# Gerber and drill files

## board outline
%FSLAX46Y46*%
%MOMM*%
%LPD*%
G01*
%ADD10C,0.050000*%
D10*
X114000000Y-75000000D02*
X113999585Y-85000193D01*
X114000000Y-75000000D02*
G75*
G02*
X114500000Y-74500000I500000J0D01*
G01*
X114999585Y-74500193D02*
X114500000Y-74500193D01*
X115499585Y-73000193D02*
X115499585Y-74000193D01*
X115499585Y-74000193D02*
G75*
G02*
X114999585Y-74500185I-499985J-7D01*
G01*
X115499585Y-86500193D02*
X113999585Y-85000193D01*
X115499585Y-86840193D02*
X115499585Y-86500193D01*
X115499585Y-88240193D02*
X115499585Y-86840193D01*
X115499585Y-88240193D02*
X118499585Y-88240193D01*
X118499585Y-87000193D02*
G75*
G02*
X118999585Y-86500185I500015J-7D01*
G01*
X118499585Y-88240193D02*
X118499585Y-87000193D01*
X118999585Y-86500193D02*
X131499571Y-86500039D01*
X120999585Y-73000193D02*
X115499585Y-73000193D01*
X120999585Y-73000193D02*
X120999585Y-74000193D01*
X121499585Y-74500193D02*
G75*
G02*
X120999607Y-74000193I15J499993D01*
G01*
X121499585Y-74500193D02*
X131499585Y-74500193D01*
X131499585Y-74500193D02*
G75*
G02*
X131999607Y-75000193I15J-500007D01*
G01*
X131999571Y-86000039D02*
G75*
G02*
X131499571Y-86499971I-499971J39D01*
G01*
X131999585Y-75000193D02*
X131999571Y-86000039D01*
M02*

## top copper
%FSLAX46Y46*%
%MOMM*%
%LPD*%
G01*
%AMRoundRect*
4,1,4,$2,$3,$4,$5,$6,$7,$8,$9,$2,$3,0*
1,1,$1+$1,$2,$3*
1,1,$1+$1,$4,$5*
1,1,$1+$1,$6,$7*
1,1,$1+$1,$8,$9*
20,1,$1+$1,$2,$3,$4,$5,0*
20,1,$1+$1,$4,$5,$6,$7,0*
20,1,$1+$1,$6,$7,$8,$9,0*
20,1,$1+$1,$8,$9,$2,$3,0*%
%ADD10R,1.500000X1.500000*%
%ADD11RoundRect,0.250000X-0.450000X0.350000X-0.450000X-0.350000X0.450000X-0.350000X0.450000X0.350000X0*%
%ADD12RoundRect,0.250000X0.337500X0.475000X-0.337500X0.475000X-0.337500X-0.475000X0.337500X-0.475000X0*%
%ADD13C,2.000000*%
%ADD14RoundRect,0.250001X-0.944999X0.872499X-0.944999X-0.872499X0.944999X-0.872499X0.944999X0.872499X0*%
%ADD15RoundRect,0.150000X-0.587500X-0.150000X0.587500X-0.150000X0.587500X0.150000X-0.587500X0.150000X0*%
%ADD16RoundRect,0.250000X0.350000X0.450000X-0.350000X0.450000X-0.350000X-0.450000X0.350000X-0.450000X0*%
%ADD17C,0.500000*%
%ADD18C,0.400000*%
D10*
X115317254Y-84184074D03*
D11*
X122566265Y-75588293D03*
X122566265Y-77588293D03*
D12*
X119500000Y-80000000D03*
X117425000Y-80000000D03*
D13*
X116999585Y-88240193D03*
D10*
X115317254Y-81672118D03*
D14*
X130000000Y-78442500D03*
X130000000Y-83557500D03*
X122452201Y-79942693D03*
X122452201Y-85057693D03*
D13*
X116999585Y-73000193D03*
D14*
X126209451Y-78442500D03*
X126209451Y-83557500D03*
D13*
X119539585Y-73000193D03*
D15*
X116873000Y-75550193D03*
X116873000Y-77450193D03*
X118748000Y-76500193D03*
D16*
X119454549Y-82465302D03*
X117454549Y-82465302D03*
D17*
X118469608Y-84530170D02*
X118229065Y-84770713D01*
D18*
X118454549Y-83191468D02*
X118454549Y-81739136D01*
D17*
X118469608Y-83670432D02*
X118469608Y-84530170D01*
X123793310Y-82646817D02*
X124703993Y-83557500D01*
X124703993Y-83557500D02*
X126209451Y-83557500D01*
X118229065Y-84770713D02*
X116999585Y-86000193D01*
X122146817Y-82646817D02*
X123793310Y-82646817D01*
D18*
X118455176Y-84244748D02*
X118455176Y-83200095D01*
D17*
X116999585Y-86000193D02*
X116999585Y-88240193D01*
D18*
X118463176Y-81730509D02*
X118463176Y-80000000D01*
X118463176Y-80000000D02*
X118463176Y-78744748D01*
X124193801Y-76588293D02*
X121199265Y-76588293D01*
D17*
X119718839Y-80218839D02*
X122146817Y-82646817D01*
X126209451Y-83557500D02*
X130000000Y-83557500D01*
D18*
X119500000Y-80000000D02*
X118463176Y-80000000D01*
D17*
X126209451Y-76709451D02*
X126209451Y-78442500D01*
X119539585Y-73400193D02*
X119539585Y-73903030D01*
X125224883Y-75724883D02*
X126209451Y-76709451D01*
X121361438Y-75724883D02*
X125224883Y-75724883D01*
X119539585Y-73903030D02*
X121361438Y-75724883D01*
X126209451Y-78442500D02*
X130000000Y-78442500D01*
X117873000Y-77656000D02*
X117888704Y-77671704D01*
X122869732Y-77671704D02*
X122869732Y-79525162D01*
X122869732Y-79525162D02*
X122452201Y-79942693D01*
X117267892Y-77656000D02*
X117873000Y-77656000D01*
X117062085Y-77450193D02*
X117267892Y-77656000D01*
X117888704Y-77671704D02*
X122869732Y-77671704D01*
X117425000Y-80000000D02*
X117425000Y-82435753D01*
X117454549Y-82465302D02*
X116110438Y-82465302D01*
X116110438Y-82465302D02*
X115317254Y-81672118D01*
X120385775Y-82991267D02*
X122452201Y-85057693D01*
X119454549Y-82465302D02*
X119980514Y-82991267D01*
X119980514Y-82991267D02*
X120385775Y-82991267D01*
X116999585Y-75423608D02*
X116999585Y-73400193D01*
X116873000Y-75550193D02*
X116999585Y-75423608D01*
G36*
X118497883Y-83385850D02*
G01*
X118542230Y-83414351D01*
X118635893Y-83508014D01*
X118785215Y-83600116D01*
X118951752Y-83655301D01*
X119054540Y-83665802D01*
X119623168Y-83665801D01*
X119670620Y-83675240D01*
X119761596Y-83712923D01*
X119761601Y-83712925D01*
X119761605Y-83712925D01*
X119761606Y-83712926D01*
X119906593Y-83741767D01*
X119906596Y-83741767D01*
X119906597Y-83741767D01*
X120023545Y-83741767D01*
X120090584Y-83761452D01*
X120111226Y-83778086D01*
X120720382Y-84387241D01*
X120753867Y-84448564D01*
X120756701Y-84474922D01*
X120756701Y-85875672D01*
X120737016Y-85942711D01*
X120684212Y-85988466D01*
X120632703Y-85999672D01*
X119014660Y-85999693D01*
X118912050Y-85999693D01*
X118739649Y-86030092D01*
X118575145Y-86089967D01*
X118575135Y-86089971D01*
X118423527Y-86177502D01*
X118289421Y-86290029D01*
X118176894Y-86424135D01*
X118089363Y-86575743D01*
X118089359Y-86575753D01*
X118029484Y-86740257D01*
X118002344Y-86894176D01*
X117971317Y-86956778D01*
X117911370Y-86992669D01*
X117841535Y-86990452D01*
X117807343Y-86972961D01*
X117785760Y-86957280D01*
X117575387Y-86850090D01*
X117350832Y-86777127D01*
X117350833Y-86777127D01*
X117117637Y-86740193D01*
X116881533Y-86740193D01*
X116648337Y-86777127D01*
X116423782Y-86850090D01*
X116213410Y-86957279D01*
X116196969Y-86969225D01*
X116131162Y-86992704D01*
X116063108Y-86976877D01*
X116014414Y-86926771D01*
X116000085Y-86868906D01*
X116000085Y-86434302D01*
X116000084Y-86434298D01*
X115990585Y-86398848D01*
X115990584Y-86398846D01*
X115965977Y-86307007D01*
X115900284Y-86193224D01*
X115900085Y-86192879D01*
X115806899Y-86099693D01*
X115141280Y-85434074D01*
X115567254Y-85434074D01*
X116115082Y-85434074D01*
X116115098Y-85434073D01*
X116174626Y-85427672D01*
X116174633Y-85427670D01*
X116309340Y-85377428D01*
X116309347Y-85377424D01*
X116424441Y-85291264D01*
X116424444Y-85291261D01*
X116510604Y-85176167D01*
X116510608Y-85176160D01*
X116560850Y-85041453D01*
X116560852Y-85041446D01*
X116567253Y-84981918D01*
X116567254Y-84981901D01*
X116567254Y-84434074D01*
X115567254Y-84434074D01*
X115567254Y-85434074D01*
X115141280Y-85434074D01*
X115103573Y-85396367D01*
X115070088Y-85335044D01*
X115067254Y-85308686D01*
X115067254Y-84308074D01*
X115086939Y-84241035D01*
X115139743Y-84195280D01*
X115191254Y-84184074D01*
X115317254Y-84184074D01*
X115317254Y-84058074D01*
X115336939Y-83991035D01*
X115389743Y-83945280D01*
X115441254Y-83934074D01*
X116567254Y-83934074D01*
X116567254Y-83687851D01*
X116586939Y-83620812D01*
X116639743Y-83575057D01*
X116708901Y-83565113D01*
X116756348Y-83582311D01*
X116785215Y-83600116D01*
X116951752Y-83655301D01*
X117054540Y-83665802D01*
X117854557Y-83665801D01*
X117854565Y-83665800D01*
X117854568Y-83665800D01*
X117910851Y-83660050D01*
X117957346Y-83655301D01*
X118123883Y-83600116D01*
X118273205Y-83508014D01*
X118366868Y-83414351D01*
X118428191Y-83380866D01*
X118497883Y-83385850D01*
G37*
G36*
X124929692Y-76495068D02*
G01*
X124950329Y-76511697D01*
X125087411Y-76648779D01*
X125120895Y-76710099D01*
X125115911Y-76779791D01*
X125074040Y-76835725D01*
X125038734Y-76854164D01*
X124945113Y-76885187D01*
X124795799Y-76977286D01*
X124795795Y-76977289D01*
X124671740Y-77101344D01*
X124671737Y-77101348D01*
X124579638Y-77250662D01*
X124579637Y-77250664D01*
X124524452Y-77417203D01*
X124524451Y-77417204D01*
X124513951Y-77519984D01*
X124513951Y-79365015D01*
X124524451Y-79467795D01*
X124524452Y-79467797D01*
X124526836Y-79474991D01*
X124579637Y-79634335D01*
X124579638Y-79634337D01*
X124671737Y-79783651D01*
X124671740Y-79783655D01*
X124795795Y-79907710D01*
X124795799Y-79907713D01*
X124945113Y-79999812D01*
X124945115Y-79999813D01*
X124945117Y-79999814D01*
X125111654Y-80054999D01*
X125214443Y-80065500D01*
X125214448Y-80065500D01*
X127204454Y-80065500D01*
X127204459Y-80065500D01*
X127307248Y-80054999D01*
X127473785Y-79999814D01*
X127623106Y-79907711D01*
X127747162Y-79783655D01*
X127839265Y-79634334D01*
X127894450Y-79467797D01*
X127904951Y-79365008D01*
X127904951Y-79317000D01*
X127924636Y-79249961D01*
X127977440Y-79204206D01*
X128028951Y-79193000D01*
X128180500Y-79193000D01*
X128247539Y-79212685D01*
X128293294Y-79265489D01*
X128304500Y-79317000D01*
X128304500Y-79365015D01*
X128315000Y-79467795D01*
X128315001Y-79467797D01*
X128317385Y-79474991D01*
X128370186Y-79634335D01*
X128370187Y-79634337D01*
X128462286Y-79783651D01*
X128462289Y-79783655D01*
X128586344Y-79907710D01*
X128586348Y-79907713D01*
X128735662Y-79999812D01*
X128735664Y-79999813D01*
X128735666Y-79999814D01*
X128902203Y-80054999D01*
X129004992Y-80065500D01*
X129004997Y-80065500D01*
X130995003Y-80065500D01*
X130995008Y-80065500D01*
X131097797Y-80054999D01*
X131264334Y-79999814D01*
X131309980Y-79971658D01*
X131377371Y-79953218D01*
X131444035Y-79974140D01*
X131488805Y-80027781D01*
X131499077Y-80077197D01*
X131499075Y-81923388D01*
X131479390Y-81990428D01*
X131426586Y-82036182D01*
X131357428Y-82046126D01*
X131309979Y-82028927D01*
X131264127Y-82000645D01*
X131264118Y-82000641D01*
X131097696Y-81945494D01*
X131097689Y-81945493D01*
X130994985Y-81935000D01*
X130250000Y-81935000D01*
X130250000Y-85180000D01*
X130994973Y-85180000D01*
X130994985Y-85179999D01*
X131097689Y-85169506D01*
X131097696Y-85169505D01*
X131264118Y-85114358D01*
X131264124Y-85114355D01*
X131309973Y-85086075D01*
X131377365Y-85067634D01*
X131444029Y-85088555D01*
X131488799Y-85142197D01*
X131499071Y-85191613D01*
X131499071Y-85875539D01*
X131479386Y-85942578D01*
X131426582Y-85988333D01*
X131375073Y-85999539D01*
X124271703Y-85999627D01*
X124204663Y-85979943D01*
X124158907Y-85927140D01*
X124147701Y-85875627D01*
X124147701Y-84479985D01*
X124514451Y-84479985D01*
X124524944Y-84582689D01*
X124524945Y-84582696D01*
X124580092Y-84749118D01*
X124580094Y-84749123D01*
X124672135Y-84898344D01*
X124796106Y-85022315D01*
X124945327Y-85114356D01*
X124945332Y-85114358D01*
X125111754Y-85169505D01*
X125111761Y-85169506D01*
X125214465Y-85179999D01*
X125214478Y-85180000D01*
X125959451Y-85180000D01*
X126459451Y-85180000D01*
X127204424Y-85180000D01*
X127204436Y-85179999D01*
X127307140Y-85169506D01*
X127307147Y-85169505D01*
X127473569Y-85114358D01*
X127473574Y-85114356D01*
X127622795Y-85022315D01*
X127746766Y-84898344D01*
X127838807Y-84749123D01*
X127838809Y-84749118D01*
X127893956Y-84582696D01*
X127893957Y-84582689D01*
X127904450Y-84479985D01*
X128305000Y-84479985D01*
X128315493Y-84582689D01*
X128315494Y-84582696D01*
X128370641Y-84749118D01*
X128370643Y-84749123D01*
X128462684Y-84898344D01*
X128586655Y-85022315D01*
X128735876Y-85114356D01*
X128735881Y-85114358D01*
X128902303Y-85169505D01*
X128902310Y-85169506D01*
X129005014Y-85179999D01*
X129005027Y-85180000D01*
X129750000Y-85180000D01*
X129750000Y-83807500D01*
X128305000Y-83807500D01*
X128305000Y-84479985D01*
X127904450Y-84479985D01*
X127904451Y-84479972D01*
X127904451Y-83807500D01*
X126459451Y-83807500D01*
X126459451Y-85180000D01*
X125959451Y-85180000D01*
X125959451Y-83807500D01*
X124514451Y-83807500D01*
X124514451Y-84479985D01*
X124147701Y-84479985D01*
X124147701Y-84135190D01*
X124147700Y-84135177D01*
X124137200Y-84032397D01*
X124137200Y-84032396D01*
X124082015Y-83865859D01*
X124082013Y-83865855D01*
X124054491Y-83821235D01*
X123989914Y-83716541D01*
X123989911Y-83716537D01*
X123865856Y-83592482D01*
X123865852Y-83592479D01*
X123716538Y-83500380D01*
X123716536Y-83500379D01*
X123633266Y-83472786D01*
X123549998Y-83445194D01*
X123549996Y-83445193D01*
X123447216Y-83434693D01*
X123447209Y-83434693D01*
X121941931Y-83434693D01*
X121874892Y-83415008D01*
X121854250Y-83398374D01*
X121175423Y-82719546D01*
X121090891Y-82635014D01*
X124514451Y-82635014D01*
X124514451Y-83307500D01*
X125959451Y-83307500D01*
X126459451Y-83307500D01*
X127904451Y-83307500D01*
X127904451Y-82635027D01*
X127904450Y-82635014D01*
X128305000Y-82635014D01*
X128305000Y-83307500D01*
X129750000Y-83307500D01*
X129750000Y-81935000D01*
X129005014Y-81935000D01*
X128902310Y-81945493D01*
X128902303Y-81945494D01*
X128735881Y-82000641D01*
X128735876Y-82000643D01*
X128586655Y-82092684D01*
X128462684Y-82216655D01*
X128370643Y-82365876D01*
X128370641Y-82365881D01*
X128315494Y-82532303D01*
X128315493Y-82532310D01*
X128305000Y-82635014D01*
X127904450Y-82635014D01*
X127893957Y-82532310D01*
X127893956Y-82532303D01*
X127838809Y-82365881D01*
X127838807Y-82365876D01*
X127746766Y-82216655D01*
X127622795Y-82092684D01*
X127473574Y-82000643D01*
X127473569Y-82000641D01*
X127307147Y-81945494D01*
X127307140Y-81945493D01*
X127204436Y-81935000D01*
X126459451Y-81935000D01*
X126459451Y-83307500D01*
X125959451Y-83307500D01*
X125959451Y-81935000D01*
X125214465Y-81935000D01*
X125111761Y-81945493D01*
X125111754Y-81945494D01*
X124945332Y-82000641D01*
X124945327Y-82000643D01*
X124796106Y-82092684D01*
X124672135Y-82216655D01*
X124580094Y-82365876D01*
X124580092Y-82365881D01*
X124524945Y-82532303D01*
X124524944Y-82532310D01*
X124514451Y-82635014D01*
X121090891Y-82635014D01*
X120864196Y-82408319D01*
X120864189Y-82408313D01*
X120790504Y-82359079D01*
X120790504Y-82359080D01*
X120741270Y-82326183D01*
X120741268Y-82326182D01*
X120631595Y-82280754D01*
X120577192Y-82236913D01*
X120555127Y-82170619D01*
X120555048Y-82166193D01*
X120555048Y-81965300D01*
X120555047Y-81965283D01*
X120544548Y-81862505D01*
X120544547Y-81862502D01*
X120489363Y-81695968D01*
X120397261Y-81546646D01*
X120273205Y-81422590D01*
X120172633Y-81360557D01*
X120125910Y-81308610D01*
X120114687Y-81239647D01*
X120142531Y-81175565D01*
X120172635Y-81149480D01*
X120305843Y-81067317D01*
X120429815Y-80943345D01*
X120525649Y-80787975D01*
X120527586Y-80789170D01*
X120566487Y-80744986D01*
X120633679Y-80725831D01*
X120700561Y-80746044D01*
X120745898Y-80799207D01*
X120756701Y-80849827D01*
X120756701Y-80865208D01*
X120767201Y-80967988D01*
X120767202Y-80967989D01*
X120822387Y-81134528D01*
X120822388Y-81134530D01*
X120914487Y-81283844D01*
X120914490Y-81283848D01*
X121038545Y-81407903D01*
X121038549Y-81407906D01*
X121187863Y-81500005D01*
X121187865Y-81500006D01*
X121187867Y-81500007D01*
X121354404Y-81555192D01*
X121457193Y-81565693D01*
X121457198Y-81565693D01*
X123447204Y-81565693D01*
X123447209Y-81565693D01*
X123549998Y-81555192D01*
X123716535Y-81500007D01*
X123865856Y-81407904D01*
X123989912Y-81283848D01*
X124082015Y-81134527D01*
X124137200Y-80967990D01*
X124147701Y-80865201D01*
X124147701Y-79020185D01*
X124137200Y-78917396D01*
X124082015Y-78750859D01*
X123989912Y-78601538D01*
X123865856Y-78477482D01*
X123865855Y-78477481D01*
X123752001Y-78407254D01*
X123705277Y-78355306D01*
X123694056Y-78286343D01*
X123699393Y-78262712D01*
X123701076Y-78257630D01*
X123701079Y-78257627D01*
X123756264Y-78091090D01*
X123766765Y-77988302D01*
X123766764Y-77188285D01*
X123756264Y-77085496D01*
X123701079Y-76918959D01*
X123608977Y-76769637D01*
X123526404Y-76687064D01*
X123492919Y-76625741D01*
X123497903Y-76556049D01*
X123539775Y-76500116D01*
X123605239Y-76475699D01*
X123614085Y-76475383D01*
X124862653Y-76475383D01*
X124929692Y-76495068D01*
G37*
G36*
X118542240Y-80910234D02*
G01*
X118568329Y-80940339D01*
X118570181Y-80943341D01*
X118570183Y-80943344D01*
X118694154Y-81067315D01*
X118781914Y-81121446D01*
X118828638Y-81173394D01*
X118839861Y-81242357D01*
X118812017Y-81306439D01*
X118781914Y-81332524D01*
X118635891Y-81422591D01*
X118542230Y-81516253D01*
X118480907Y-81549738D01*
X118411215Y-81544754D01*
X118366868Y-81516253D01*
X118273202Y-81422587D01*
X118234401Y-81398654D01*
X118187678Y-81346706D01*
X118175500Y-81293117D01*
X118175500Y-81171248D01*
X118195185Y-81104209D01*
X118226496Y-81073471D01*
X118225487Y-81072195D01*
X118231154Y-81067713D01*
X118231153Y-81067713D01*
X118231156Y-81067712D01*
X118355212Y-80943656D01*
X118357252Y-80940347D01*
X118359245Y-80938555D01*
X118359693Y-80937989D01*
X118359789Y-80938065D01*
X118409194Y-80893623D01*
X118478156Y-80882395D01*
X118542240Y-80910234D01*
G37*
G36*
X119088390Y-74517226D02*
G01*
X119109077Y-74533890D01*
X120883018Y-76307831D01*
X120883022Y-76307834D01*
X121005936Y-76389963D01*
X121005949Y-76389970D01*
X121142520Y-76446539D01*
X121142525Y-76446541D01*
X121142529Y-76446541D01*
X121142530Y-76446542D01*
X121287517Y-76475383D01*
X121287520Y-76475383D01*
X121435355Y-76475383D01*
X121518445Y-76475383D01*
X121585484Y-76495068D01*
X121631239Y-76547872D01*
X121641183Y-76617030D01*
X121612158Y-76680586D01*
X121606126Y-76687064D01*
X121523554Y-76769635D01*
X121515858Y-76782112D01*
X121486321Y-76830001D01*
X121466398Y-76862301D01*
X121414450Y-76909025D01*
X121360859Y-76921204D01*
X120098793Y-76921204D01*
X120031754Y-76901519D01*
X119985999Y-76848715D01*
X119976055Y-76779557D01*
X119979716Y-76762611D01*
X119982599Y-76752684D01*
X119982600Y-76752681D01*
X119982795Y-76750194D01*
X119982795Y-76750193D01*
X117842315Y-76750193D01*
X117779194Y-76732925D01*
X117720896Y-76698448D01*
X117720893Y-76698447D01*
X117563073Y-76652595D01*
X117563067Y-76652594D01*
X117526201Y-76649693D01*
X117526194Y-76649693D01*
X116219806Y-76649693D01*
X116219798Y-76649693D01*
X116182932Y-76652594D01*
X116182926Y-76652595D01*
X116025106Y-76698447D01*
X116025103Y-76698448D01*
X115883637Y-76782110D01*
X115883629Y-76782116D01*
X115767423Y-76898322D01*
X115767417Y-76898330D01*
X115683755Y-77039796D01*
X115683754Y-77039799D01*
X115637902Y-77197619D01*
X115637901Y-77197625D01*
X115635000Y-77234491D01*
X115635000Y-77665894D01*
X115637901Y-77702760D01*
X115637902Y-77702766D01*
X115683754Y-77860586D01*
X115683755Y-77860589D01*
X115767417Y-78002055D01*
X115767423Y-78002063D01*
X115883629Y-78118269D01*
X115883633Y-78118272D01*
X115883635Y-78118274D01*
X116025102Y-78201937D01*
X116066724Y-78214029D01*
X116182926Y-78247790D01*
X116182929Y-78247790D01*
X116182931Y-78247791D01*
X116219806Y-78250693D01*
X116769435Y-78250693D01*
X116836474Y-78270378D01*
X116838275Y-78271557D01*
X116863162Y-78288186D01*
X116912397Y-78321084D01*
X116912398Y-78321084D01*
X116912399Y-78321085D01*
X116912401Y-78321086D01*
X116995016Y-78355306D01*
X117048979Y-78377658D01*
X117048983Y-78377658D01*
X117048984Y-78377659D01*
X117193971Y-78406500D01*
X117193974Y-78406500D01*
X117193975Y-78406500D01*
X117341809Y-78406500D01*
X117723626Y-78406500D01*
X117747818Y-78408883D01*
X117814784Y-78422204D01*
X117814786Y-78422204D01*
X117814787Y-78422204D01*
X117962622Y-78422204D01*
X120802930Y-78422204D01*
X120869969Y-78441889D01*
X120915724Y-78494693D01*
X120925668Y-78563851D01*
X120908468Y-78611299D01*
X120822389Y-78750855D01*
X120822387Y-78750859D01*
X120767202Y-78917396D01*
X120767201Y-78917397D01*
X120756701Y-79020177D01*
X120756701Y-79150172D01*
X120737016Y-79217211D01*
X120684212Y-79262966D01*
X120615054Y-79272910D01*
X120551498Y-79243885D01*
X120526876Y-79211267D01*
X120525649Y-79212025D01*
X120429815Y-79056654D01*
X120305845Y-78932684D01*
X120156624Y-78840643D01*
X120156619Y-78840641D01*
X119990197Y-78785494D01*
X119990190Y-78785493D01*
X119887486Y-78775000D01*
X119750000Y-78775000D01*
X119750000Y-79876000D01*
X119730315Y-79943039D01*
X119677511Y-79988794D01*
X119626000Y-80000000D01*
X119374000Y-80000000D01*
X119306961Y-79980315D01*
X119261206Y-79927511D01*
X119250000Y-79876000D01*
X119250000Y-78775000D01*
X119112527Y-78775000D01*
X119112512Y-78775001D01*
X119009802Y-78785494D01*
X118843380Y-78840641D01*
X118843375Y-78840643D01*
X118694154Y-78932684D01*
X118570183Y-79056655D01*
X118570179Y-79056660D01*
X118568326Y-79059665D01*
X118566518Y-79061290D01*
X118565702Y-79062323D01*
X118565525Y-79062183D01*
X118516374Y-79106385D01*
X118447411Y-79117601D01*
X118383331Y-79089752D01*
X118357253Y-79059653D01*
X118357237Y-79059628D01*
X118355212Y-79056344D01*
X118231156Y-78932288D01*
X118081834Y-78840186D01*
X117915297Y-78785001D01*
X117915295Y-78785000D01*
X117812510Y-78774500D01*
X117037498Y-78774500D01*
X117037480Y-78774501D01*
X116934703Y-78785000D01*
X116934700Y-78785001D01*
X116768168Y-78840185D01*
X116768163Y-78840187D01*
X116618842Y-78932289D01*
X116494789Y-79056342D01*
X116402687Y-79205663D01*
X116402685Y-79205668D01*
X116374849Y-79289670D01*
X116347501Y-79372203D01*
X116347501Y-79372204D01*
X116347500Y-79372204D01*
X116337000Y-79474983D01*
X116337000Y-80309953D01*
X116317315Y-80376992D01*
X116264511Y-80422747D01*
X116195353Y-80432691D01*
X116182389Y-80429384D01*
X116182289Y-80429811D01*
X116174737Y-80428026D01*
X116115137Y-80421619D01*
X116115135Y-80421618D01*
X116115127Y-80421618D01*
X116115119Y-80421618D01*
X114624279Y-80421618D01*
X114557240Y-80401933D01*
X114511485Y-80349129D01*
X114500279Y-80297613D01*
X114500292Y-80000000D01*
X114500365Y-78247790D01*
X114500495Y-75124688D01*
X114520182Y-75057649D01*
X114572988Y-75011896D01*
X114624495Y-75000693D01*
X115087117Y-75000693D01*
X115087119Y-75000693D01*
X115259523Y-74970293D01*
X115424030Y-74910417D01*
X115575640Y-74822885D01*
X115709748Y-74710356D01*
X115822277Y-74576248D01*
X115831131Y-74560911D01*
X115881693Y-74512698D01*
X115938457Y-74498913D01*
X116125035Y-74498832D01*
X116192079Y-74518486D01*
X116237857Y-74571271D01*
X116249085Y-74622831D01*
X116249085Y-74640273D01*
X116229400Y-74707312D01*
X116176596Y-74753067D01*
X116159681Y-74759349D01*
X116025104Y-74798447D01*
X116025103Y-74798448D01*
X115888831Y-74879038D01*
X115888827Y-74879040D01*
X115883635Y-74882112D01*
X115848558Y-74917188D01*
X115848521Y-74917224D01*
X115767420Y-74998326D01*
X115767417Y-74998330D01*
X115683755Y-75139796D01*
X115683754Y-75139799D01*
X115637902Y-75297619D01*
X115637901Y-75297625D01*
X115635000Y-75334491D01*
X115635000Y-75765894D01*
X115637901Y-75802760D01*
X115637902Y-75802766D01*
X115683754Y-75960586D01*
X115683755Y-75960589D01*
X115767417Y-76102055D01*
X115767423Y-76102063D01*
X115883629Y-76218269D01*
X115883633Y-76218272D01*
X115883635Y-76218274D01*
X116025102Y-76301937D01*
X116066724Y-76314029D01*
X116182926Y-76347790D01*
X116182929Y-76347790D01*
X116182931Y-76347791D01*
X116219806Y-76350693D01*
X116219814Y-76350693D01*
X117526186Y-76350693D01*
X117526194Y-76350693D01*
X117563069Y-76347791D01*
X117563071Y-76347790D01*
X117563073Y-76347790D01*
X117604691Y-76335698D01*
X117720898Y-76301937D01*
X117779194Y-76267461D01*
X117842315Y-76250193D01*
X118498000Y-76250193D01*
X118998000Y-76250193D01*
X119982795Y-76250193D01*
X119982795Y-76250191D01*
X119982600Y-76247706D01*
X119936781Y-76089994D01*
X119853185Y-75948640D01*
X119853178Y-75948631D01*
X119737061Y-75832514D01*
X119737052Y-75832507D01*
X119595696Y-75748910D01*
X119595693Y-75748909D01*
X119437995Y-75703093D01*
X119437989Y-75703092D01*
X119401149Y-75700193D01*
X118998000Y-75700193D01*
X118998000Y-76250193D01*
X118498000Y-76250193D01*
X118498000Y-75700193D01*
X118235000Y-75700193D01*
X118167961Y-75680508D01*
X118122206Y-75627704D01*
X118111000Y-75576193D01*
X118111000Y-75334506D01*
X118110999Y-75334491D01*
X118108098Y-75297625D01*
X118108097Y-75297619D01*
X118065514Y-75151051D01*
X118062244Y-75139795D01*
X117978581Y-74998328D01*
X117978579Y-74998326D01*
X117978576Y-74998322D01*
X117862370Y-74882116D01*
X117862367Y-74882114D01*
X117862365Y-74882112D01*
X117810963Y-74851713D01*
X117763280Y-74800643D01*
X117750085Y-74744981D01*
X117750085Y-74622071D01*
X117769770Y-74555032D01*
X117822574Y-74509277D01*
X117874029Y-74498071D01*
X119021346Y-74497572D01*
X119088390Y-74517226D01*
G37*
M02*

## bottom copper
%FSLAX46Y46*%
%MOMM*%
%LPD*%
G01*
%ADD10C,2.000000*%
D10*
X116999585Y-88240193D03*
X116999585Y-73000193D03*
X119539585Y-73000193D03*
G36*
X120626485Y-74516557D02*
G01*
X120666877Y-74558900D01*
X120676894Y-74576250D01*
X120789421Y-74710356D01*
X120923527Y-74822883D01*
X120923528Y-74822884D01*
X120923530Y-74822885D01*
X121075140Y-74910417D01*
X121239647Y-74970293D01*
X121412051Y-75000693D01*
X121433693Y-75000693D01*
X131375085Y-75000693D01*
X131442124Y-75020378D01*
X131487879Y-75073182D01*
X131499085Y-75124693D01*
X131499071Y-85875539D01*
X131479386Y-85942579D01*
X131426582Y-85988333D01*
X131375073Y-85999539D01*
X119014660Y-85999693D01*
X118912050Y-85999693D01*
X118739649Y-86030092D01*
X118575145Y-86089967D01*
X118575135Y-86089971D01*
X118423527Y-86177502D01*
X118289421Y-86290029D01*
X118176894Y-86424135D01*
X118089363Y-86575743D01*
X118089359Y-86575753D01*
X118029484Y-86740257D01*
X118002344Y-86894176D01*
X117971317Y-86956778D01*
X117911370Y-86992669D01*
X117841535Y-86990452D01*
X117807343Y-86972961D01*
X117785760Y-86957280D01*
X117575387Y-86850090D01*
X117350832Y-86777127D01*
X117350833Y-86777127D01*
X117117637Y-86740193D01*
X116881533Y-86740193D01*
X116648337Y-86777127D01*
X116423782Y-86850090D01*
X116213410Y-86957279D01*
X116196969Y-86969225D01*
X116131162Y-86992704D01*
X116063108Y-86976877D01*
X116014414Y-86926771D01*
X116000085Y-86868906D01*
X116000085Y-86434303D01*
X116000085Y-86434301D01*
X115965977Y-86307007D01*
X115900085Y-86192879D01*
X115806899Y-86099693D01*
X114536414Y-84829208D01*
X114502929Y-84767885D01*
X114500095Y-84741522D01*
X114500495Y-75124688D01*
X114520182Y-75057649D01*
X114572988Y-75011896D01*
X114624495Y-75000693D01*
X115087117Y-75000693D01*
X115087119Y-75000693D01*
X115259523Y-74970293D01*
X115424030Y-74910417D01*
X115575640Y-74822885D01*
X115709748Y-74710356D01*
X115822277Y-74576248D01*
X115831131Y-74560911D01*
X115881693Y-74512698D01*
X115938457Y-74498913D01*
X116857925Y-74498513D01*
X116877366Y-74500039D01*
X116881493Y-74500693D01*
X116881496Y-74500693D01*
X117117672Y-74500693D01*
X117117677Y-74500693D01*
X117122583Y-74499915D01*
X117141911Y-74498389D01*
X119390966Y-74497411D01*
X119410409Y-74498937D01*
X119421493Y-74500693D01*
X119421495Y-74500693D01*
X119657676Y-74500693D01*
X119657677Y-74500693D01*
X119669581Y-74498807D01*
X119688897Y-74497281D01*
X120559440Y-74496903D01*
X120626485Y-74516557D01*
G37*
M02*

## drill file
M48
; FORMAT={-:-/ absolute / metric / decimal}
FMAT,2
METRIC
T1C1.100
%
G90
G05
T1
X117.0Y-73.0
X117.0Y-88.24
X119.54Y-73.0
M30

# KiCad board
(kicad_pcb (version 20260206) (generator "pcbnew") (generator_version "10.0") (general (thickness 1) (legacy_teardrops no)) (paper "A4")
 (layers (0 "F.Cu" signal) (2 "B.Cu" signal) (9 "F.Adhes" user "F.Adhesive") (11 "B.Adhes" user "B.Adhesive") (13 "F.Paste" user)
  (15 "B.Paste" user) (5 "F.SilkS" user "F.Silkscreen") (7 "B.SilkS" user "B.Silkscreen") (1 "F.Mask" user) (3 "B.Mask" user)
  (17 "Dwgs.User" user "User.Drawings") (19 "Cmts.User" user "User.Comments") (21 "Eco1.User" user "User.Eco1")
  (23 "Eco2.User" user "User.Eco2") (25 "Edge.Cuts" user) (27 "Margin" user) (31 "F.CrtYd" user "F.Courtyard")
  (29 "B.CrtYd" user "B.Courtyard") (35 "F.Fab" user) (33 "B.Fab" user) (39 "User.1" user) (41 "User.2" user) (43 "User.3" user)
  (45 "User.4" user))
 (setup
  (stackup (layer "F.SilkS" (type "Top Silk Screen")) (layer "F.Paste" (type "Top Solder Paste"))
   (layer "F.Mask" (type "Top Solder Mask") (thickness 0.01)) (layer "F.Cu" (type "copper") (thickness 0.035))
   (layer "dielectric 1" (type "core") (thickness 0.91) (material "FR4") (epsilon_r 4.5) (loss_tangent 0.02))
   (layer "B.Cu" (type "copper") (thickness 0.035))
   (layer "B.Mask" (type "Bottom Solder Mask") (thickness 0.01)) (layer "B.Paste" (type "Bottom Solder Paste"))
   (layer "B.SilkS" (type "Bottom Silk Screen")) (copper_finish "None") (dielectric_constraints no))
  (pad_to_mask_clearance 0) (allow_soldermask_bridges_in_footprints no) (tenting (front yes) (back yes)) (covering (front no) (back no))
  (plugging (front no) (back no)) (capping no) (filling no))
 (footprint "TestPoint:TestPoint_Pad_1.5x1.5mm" (layer "F.Cu") (at 115.317254 84.184074)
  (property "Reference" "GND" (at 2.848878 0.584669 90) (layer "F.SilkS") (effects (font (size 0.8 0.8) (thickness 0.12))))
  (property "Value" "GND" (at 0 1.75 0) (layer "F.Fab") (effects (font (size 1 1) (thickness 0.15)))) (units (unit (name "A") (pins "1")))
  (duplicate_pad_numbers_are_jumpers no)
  (pad "1" smd rect (at 0 0) (size 1.5 1.5) (layers "F.Cu" "F.Mask") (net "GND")))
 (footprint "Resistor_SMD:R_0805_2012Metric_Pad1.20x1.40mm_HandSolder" (layer "F.Cu") (at 122.566265 76.588293 -90)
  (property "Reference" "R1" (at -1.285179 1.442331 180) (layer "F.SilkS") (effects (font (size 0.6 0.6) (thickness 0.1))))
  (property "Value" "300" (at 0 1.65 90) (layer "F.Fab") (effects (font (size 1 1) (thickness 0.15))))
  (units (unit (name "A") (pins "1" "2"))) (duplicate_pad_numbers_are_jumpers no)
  (pad "1" smd roundrect (at -1 0 270) (size 1.2 1.4) (layers "F.Cu" "F.Mask" "F.Paste") (roundrect_rratio 0.208333) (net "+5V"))
  (pad "2" smd roundrect (at 1 0 270) (size 1.2 1.4) (layers "F.Cu" "F.Mask" "F.Paste") (roundrect_rratio 0.208333) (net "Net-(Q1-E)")))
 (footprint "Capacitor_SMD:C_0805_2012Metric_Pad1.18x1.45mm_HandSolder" (layer "F.Cu") (at 118.4625 80 180)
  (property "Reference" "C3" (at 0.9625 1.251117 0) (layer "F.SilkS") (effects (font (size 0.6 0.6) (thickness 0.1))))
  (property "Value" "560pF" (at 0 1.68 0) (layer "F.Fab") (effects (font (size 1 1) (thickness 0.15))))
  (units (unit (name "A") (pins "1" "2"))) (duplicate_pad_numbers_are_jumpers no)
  (pad "1" smd roundrect (at -1.0375 0 180) (size 1.175 1.45) (layers "F.Cu" "F.Mask" "F.Paste") (roundrect_rratio 0.212766) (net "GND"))
  (pad "2" smd roundrect (at 1.0375 0 180) (size 1.175 1.45) (layers "F.Cu" "F.Mask" "F.Paste") (roundrect_rratio 0.212766)
   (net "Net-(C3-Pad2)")))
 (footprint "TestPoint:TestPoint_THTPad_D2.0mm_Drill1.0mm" (layer "F.Cu") (at 116.999585 88.240193 -90)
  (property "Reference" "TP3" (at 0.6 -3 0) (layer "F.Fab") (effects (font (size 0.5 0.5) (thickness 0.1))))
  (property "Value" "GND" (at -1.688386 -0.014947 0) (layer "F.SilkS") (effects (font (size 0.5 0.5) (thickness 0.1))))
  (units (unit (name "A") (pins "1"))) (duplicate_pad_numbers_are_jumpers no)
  (pad "1" thru_hole circle (at 0 0 270) (size 2 2) (drill 1.1) (layers "*.Cu" "*.Mask") (remove_unused_layers no) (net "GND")))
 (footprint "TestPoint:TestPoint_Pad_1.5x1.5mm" (layer "F.Cu") (at 115.317254 81.672118 -90)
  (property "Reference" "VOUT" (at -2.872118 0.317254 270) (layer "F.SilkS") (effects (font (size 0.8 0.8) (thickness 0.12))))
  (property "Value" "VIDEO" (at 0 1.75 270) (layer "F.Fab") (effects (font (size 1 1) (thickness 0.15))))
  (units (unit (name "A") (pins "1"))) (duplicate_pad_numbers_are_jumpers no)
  (pad "1" smd rect (at 0 0 270) (size 1.5 1.5) (layers "F.Cu" "F.Mask") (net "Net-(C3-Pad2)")))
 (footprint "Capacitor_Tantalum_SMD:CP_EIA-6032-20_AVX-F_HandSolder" (layer "F.Cu") (at 130 81 -90)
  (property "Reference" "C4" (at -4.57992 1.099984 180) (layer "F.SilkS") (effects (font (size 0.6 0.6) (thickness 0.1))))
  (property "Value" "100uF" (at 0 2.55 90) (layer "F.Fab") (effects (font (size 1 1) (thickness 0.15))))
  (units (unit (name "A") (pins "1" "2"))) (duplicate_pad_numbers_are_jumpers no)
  (pad "1" smd roundrect (at -2.5575 0 270) (size 2.245 2.39) (layers "F.Cu" "F.Mask" "F.Paste") (roundrect_rratio 0.111359) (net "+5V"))
  (pad "2" smd roundrect (at 2.5575 0 270) (size 2.245 2.39) (layers "F.Cu" "F.Mask" "F.Paste") (roundrect_rratio 0.111359) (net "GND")))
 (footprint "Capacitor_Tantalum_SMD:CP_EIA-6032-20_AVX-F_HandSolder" (layer "F.Cu") (at 122.452201 82.500193 -90)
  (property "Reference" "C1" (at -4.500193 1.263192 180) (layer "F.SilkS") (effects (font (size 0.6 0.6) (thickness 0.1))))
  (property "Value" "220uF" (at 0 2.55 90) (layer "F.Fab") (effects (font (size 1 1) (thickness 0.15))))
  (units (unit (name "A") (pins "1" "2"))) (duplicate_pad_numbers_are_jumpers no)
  (pad "1" smd roundrect (at -2.5575 0 270) (size 2.245 2.39) (layers "F.Cu" "F.Mask" "F.Paste") (roundrect_rratio 0.111359)
   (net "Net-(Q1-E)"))
  (pad "2" smd roundrect (at 2.5575 0 270) (size 2.245 2.39) (layers "F.Cu" "F.Mask" "F.Paste") (roundrect_rratio 0.111359)
   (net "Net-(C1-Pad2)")))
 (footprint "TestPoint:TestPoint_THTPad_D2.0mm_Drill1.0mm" (layer "F.Cu") (at 116.999585 73.000193 -90)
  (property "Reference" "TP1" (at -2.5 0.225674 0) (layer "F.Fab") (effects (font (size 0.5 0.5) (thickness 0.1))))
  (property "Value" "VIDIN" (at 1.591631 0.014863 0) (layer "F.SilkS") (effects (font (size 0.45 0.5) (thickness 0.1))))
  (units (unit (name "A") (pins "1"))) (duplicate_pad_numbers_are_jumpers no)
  (pad "1" thru_hole circle (at 0 0 270) (size 2 2) (drill 1.1) (layers "*.Cu" "*.Mask") (remove_unused_layers no) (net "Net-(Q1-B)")))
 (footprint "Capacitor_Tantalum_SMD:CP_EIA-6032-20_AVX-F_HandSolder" (layer "F.Cu") (at 126.209451 81 -90)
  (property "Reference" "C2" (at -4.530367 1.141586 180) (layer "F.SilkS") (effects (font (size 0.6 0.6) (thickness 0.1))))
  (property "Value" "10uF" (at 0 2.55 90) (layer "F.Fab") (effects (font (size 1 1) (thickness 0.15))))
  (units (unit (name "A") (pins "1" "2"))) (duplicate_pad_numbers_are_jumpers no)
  (pad "1" smd roundrect (at -2.5575 0 270) (size 2.245 2.39) (layers "F.Cu" "F.Mask" "F.Paste") (roundrect_rratio 0.111359) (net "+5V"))
  (pad "2" smd roundrect (at 2.5575 0 270) (size 2.245 2.39) (layers "F.Cu" "F.Mask" "F.Paste") (roundrect_rratio 0.111359) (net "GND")))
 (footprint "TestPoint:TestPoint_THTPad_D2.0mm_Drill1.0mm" (layer "F.Cu") (at 119.539585 73.000193 -90)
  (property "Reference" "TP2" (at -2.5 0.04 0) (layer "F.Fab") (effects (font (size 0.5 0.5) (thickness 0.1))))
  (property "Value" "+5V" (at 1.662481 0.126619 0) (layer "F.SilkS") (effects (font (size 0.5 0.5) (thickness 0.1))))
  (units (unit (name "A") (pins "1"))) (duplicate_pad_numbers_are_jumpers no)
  (pad "1" thru_hole circle (at 0 0 270) (size 2 2) (drill 1.1) (layers "*.Cu" "*.Mask") (remove_unused_layers no) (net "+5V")))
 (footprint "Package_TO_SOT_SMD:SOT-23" (layer "F.Cu") (at 117.8105 76.500193)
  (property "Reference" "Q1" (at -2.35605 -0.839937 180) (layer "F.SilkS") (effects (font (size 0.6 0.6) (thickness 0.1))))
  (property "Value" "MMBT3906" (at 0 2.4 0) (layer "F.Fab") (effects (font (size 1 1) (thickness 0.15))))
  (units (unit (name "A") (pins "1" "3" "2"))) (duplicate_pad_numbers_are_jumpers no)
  (pad "1" smd roundrect (at -0.9375 -0.95) (size 1.475 0.6) (layers "F.Cu" "F.Mask" "F.Paste") (roundrect_rratio 0.25) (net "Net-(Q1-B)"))
  (pad "2" smd roundrect (at -0.9375 0.95) (size 1.475 0.6) (layers "F.Cu" "F.Mask" "F.Paste") (roundrect_rratio 0.25) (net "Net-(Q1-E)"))
  (pad "3" smd roundrect (at 0.9375 0) (size 1.475 0.6) (layers "F.Cu" "F.Mask" "F.Paste") (roundrect_rratio 0.25) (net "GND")))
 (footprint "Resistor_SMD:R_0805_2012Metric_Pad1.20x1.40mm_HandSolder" (layer "F.Cu") (at 118.454549 82.465302 180)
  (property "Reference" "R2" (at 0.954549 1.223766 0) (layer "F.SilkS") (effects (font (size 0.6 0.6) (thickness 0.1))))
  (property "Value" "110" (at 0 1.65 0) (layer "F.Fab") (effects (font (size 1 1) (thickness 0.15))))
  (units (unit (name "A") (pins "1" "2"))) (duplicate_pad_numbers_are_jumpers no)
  (pad "1" smd roundrect (at -1 0 180) (size 1.2 1.4) (layers "F.Cu" "F.Mask" "F.Paste") (roundrect_rratio 0.208333) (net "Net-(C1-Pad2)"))
  (pad "2" smd roundrect (at 1 0 180) (size 1.2 1.4) (layers "F.Cu" "F.Mask" "F.Paste") (roundrect_rratio 0.208333) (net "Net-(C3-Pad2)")))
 (gr_line (start 114 75) (end 113.999585 85.000193) (stroke (width 0.05) (type default)) (layer "Edge.Cuts"))
 (gr_arc (start 114 75) (mid 114.146447 74.646447) (end 114.5 74.5) (stroke (width 0.05) (type default)) (layer "Edge.Cuts"))
 (gr_line (start 114.999585 74.500193) (end 114.5 74.500193) (stroke (width 0.05) (type default)) (layer "Edge.Cuts"))
 (gr_line (start 115.499585 73.000193) (end 115.499585 74.000193) (stroke (width 0.05) (type default)) (layer "Edge.Cuts"))
 (gr_arc (start 115.499585 74.000193) (mid 115.353138 74.353746) (end 114.999585 74.500193) (stroke (width 0.05) (type default))
  (layer "Edge.Cuts"))
 (gr_line (start 115.499585 86.500193) (end 113.999585 85.000193) (stroke (width 0.05) (type default)) (layer "Edge.Cuts"))
 (gr_line (start 115.499585 86.840193) (end 115.499585 86.500193) (stroke (width 0.05) (type default)) (layer "Edge.Cuts"))
 (gr_line (start 115.499585 88.240193) (end 115.499585 86.840193) (stroke (width 0.05) (type default)) (layer "Edge.Cuts"))
 (gr_line (start 115.499585 88.240193) (end 118.499585 88.240193) (stroke (width 0.05) (type default)) (layer "Edge.Cuts"))
 (gr_arc (start 118.499585 87.000193) (mid 118.646032 86.64664) (end 118.999585 86.500193) (stroke (width 0.05) (type default))
  (layer "Edge.Cuts"))
 (gr_line (start 118.499585 88.240193) (end 118.499585 87.000193) (stroke (width 0.05) (type default)) (layer "Edge.Cuts"))
 (gr_line (start 118.999585 86.500193) (end 131.499571 86.500039) (stroke (width 0.05) (type default)) (layer "Edge.Cuts"))
 (gr_line (start 120.999585 73.000193) (end 115.499585 73.000193) (stroke (width 0.05) (type default)) (layer "Edge.Cuts"))
 (gr_line (start 120.999585 73.000193) (end 120.999585 74.000193) (stroke (width 0.05) (type default)) (layer "Edge.Cuts"))
 (gr_arc (start 121.499585 74.500193) (mid 121.146032 74.353746) (end 120.999585 74.000193) (stroke (width 0.05) (type default))
  (layer "Edge.Cuts"))
 (gr_line (start 121.499585 74.500193) (end 131.499585 74.500193) (stroke (width 0.05) (type default)) (layer "Edge.Cuts"))
 (gr_arc (start 131.499585 74.500193) (mid 131.853138 74.64664) (end 131.999585 75.000193) (stroke (width 0.05) (type default))
  (layer "Edge.Cuts"))
 (gr_arc (start 131.999571 86.000039) (mid 131.853124 86.353592) (end 131.499571 86.500039) (stroke (width 0.05) (type default))
  (layer "Edge.Cuts"))
 (gr_line (start 131.999585 75.000193) (end 131.999571 86.000039) (stroke (width 0.05) (type default)) (layer "Edge.Cuts"))
 (segment (start 118.469608 84.53017) (end 118.229065 84.770713) (width 0.5) (layer "F.Cu") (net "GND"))
 (segment (start 118.454549 83.191468) (end 118.454549 81.739136) (width 0.4) (layer "F.Cu") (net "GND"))
 (segment (start 118.469608 83.670432) (end 118.469608 84.53017) (width 0.5) (layer "F.Cu") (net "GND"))
 (segment (start 123.79331 82.646817) (end 124.703993 83.5575) (width 0.5) (layer "F.Cu") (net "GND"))
 (segment (start 124.703993 83.5575) (end 126.209451 83.5575) (width 0.5) (layer "F.Cu") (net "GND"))
 (segment (start 118.229065 84.770713) (end 116.999585 86.000193) (width 0.5) (layer "F.Cu") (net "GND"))
 (segment (start 122.146817 82.646817) (end 123.79331 82.646817) (width 0.5) (layer "F.Cu") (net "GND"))
 (segment (start 118.455176 84.244748) (end 118.455176 83.200095) (width 0.4) (layer "F.Cu") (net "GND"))
 (segment (start 116.999585 86.000193) (end 116.999585 88.240193) (width 0.5) (layer "F.Cu") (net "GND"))
 (segment (start 118.463176 81.730509) (end 118.463176 80) (width 0.4) (layer "F.Cu") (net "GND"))
 (segment (start 118.463176 80) (end 118.463176 78.744748) (width 0.4) (layer "F.Cu") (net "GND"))
 (segment (start 124.193801 76.588293) (end 121.199265 76.588293) (width 0.4) (layer "F.Cu") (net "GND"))
 (segment (start 119.718839 80.218839) (end 122.146817 82.646817) (width 0.5) (layer "F.Cu") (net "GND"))
 (segment (start 126.209451 83.5575) (end 130 83.5575) (width 0.5) (layer "F.Cu") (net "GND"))
 (segment (start 119.5 80) (end 118.463176 80) (width 0.4) (layer "F.Cu") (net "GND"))
 (segment (start 126.209451 76.709451) (end 126.209451 78.4425) (width 0.5) (layer "F.Cu") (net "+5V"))
 (segment (start 119.539585 73.400193) (end 119.539585 73.90303) (width 0.5) (layer "F.Cu") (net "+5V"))
 (segment (start 125.224883 75.724883) (end 126.209451 76.709451) (width 0.5) (layer "F.Cu") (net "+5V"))
 (segment (start 121.361438 75.724883) (end 125.224883 75.724883) (width 0.5) (layer "F.Cu") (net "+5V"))
 (segment (start 119.539585 73.90303) (end 121.361438 75.724883) (width 0.5) (layer "F.Cu") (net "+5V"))
 (segment (start 126.209451 78.4425) (end 130 78.4425) (width 0.5) (layer "F.Cu") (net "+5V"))
 (segment (start 117.873 77.656) (end 117.888704 77.671704) (width 0.5) (layer "F.Cu") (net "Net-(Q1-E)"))
 (segment (start 122.869732 77.671704) (end 122.869732 79.525162) (width 0.5) (layer "F.Cu") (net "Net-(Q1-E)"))
 (segment (start 122.869732 79.525162) (end 122.452201 79.942693) (width 0.5) (layer "F.Cu") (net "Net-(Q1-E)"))
 (segment (start 117.267892 77.656) (end 117.873 77.656) (width 0.5) (layer "F.Cu") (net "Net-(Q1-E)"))
 (segment (start 117.062085 77.450193) (end 117.267892 77.656) (width 0.5) (layer "F.Cu") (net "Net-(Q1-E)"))
 (segment (start 117.888704 77.671704) (end 122.869732 77.671704) (width 0.5) (layer "F.Cu") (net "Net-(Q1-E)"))
 (segment (start 117.425 80) (end 117.425 82.435753) (width 0.5) (layer "F.Cu") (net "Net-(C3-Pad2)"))
 (segment (start 117.454549 82.465302) (end 116.110438 82.465302) (width 0.5) (layer "F.Cu") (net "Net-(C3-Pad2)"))
 (segment (start 116.110438 82.465302) (end 115.317254 81.672118) (width 0.5) (layer "F.Cu") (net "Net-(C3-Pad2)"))
 (segment (start 120.385775 82.991267) (end 122.452201 85.057693) (width 0.5) (layer "F.Cu") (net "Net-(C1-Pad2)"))
 (segment (start 119.454549 82.465302) (end 119.980514 82.991267) (width 0.5) (layer "F.Cu") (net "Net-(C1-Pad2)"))
 (segment (start 119.980514 82.991267) (end 120.385775 82.991267) (width 0.5) (layer "F.Cu") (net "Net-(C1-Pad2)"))
 (segment (start 116.999585 75.423608) (end 116.999585 73.400193) (width 0.5) (layer "F.Cu") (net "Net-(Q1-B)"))
 (segment (start 116.873 75.550193) (end 116.999585 75.423608) (width 0.5) (layer "F.Cu") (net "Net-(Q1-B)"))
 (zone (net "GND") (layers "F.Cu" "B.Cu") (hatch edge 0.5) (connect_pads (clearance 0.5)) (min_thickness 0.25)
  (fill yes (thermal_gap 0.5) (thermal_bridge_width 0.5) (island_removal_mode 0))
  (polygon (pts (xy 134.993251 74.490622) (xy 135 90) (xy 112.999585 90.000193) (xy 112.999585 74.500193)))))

